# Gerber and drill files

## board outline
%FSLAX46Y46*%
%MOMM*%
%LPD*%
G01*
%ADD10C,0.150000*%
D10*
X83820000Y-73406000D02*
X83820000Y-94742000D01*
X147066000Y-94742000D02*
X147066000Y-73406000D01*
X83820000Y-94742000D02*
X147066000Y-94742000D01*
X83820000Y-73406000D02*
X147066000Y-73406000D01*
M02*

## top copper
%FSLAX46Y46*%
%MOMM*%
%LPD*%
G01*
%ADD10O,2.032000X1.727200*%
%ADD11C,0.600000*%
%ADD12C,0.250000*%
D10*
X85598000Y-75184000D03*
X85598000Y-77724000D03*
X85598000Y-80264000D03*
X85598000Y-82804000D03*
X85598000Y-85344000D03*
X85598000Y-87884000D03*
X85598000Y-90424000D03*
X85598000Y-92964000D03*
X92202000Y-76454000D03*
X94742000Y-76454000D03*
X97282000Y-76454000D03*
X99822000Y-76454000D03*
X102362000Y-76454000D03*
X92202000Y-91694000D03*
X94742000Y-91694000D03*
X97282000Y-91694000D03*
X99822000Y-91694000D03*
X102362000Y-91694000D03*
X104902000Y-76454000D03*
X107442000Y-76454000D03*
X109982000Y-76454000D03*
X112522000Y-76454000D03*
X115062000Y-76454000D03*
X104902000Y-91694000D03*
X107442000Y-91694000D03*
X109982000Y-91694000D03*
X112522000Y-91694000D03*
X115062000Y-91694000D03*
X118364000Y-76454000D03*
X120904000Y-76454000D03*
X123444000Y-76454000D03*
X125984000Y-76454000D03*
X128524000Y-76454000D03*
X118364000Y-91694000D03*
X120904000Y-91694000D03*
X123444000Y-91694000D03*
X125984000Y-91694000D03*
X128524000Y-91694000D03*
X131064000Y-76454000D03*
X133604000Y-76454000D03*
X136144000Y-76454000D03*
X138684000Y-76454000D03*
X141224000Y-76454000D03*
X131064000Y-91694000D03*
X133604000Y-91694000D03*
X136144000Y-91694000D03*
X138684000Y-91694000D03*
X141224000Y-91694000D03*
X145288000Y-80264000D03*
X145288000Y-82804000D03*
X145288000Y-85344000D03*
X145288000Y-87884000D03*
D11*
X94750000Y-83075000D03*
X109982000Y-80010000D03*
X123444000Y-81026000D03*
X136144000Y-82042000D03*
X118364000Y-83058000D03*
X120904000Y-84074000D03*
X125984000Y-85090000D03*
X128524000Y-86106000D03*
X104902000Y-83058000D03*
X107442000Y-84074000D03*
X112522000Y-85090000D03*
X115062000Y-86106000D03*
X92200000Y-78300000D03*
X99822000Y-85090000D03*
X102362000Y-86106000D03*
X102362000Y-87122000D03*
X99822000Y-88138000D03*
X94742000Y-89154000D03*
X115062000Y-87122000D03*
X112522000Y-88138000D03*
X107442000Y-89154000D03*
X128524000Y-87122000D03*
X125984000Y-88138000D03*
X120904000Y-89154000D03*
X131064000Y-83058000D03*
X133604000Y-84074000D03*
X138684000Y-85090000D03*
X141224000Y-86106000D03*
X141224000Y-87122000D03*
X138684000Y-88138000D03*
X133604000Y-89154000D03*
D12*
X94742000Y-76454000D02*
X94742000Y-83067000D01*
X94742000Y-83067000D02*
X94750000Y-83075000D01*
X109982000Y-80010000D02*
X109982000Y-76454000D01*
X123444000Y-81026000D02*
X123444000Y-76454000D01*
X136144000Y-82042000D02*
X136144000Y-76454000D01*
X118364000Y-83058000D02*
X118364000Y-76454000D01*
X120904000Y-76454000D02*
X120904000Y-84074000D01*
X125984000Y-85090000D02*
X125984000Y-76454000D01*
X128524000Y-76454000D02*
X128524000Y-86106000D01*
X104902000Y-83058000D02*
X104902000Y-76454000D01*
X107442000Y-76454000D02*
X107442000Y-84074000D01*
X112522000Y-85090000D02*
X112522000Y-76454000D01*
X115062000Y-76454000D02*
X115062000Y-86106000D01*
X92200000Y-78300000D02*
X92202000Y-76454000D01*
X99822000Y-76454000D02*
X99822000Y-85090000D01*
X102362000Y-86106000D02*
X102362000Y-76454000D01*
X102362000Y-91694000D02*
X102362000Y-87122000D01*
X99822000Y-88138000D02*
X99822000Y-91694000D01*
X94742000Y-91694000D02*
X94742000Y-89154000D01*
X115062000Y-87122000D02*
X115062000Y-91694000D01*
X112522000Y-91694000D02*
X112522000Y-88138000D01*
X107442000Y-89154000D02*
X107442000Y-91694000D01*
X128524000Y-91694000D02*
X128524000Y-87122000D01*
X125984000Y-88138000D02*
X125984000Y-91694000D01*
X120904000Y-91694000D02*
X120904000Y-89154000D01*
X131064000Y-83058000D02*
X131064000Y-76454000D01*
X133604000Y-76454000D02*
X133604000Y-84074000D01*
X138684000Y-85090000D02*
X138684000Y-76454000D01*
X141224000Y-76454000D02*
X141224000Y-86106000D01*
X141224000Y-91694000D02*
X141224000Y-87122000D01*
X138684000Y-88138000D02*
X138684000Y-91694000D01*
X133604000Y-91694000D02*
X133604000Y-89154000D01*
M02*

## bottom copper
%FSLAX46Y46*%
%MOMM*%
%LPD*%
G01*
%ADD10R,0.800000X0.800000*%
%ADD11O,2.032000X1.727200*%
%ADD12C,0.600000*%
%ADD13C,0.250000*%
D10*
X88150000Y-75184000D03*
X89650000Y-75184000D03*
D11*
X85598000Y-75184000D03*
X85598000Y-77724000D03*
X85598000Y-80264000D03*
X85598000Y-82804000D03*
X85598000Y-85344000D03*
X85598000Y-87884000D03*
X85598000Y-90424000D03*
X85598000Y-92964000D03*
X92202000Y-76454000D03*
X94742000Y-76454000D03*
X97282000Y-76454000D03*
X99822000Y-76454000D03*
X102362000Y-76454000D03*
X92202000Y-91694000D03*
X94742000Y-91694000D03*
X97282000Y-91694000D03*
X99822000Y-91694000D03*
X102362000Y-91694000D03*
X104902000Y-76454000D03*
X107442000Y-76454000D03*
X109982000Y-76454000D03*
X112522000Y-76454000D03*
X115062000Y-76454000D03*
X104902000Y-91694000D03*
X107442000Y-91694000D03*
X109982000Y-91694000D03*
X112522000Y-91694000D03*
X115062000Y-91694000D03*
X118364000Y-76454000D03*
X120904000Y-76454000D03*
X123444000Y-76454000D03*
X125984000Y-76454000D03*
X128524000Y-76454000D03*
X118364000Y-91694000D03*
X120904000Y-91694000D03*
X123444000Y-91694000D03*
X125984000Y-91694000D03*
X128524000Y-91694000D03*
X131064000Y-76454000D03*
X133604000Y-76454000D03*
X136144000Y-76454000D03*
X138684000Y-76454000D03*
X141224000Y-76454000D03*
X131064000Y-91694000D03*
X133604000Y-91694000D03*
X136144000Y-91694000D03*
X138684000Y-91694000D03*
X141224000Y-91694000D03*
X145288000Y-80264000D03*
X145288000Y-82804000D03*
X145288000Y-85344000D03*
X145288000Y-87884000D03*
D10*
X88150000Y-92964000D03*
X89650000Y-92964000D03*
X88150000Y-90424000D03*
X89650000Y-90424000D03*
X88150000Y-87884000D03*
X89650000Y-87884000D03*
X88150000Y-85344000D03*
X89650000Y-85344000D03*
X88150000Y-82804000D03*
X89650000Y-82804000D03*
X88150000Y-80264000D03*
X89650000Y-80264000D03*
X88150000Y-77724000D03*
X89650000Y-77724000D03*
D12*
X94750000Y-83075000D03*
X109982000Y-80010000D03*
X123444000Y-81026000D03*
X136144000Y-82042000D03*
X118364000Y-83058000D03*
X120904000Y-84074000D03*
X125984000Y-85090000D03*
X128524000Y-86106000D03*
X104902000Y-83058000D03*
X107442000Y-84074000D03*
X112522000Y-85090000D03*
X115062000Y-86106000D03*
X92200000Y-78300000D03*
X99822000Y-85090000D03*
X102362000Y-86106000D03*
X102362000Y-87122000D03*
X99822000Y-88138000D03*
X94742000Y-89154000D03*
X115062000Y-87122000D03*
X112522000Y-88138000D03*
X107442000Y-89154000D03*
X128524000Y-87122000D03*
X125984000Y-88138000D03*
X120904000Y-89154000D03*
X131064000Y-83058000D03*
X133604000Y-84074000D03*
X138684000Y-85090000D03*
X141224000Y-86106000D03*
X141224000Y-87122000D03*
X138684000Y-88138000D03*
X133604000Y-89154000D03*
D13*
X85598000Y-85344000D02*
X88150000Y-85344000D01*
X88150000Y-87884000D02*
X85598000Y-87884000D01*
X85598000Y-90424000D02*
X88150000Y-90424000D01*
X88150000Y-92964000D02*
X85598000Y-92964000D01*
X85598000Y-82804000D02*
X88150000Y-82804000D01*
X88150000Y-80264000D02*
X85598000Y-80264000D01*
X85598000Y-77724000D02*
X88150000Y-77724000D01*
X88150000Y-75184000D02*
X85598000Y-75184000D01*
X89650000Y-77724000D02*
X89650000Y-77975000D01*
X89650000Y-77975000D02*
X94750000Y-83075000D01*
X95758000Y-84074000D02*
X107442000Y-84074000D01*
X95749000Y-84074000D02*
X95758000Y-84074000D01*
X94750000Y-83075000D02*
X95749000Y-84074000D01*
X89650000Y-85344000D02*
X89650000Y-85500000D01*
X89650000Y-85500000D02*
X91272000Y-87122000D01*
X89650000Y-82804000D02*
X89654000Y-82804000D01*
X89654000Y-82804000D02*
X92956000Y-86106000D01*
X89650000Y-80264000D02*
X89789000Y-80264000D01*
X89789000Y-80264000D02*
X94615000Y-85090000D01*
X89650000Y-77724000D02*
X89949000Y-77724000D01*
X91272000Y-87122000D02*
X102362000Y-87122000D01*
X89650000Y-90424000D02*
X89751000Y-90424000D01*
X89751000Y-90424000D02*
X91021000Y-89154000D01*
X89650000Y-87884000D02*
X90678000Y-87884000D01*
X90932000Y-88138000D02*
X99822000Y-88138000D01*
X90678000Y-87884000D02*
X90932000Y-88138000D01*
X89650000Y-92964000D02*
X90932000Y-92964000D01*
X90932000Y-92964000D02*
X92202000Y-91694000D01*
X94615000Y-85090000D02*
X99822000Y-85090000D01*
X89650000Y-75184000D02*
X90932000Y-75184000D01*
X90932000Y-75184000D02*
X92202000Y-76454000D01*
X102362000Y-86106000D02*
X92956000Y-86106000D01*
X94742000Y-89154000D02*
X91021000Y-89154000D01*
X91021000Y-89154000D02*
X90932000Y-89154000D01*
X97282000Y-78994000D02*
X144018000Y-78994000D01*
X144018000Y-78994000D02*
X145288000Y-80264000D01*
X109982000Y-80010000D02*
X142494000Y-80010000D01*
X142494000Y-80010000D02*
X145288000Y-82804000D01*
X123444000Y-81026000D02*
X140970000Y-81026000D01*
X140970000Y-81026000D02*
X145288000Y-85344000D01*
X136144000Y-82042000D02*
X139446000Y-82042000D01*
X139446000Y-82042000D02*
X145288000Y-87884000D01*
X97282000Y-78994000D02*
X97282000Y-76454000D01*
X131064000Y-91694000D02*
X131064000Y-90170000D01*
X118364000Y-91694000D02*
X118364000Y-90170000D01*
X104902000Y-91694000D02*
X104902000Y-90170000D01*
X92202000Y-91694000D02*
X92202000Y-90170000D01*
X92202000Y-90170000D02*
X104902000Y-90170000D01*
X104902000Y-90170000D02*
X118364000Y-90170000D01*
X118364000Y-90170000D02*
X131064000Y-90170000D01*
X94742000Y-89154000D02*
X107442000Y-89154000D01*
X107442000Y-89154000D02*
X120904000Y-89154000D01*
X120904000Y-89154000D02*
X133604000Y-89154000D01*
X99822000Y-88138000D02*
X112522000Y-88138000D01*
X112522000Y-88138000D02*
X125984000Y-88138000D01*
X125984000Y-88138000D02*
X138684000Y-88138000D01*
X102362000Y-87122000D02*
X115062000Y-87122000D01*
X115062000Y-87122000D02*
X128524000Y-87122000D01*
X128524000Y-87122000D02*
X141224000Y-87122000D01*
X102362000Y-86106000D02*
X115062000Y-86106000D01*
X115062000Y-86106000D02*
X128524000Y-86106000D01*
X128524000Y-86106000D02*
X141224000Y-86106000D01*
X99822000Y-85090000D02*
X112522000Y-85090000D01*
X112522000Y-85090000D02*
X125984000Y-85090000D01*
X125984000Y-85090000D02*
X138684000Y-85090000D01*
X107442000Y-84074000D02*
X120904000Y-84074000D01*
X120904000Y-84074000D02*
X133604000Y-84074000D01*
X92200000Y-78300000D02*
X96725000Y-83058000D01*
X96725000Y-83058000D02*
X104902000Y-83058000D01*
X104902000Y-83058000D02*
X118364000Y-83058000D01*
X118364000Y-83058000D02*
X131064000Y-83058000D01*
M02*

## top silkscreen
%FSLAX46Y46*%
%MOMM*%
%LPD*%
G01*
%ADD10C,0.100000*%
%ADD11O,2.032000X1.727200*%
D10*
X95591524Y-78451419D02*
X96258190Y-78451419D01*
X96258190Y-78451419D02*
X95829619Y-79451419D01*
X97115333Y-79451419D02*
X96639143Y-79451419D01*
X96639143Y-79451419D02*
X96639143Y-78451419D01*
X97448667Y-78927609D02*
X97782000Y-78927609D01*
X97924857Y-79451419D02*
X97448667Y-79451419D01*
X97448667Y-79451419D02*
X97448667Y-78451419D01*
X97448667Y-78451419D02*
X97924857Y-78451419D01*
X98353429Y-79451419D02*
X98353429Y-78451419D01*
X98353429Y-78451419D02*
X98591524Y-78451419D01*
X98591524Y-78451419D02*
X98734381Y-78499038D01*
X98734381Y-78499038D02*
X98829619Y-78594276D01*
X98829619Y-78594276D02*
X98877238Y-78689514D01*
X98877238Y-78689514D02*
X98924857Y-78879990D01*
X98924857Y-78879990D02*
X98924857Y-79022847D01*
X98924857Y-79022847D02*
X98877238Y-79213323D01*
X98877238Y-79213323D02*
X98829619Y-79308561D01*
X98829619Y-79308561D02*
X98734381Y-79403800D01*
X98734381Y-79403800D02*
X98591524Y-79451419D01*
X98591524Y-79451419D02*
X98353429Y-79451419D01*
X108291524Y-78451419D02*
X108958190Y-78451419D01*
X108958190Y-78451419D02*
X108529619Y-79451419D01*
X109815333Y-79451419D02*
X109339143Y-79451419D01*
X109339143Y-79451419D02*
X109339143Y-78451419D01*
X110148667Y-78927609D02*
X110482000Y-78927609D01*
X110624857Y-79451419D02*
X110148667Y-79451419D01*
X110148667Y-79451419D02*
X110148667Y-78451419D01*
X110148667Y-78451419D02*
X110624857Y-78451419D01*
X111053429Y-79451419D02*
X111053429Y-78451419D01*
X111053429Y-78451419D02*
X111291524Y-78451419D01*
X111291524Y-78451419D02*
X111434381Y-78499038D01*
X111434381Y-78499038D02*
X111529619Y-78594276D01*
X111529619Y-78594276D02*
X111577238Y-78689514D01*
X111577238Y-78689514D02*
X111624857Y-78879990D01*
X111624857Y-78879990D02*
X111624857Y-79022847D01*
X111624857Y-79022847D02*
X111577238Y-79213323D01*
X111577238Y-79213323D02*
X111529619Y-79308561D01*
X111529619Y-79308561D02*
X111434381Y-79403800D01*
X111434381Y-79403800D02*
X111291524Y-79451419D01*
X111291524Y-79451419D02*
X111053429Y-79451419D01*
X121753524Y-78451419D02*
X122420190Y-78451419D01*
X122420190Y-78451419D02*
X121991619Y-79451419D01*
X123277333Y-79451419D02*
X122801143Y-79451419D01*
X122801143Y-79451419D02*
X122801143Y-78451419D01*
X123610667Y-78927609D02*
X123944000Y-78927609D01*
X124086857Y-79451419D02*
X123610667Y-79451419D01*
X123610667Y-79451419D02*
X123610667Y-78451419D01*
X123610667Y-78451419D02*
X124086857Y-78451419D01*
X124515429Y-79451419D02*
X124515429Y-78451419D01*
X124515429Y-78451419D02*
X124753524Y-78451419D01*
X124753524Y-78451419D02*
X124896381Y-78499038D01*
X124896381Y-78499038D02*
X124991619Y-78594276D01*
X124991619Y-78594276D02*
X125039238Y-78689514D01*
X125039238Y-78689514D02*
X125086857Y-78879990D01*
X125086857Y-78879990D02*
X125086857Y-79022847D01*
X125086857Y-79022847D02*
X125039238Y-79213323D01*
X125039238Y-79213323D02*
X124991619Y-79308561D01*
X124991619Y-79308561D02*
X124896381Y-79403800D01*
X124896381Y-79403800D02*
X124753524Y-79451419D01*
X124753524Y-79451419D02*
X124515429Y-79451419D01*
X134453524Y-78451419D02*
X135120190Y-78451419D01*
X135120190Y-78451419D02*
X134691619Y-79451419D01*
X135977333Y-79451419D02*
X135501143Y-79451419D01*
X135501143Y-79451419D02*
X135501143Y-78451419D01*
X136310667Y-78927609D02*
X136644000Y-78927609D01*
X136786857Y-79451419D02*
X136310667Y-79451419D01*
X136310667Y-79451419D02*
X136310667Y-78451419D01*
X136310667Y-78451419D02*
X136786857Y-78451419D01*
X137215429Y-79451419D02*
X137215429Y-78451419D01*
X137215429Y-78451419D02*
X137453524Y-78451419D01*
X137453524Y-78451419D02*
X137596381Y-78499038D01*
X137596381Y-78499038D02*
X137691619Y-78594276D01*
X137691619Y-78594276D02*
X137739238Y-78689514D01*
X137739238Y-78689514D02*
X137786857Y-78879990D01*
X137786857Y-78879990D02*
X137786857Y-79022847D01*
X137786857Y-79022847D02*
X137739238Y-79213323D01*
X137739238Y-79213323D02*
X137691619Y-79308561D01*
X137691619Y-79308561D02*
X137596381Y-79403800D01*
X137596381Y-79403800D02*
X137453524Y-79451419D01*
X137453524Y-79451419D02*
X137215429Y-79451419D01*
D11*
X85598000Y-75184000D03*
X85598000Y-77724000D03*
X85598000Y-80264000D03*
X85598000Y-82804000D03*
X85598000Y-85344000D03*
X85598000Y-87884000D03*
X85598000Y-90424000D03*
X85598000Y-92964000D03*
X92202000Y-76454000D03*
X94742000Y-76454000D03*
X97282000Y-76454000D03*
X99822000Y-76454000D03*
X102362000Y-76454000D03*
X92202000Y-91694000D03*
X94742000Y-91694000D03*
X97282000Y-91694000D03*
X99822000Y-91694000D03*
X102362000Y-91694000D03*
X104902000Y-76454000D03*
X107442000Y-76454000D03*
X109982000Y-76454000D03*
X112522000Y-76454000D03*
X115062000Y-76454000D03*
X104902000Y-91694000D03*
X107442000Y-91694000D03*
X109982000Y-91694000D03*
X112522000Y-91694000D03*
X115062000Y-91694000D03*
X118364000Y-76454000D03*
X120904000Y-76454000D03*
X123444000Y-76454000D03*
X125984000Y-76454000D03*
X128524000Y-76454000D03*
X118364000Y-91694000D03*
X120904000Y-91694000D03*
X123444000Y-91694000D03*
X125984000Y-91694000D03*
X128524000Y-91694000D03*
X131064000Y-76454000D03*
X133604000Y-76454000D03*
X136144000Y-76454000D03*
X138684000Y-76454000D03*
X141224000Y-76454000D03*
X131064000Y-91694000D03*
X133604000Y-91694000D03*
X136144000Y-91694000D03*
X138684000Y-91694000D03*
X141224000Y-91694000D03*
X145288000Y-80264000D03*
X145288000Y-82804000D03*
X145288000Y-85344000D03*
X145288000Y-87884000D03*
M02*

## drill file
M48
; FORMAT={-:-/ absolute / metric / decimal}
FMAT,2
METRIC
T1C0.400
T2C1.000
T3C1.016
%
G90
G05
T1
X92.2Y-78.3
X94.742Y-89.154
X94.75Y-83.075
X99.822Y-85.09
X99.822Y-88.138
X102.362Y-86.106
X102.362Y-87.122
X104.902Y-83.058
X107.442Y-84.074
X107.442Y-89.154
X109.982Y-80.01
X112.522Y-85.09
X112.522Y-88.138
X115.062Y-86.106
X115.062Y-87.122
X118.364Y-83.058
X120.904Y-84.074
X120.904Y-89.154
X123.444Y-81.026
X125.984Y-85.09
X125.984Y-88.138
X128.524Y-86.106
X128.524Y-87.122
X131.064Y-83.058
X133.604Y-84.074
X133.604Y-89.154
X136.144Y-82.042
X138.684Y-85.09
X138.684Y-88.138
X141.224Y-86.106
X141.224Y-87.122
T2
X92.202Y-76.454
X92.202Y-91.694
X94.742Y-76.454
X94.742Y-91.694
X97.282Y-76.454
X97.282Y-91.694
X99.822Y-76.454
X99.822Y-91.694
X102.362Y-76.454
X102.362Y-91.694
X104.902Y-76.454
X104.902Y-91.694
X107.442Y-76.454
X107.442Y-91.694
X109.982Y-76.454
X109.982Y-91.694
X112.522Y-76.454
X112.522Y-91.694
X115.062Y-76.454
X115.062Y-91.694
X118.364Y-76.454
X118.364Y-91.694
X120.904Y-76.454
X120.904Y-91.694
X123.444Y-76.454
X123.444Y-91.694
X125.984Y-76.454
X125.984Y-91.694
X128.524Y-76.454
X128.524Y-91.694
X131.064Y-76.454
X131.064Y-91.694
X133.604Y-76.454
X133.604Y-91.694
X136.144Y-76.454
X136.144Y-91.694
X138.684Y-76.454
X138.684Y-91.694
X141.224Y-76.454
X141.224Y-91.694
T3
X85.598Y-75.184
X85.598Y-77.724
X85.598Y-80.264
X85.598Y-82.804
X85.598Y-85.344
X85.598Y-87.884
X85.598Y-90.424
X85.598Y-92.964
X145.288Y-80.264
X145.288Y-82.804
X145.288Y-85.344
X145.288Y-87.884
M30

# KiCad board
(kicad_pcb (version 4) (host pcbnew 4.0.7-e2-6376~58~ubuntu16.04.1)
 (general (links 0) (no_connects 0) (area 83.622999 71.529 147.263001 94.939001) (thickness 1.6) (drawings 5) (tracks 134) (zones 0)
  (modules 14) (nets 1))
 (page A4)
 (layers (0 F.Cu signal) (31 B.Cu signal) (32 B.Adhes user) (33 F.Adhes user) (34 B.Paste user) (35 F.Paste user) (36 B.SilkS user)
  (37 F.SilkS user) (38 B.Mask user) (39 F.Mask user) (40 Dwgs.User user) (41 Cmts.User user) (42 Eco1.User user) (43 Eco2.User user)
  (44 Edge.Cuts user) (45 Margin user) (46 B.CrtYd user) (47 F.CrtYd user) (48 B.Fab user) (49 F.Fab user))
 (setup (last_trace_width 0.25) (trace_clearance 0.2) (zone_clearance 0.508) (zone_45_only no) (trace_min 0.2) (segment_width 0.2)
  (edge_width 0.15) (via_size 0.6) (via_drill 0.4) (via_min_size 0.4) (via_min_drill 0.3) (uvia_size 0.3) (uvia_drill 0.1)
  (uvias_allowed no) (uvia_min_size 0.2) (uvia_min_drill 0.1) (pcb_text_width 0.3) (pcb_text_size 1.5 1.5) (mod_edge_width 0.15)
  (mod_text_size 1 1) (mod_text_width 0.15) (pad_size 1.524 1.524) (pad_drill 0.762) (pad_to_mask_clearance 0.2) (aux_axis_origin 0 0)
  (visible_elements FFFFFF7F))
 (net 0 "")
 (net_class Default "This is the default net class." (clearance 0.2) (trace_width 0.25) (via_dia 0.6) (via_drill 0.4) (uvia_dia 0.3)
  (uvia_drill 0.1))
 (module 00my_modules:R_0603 (layer B.Cu) (at 88.9 75.184)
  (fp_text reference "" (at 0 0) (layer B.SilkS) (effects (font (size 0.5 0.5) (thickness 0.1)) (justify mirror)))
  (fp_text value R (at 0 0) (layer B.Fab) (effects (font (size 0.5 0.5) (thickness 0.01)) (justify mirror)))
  (pad 1 smd rect (at -0.75 0) (size 0.8 0.8) (layers B.Cu B.Paste B.Mask))
  (pad 2 smd rect (at 0.75 0) (size 0.8 0.8) (layers B.Cu B.Paste B.Mask)))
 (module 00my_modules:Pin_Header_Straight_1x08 (layer F.Cu) (at 85.598 75.184)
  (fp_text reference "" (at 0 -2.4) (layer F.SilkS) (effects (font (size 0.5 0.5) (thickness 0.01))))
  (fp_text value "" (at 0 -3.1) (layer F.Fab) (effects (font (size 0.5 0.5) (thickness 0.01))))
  (pad 1 thru_hole oval (at 0 0) (size 2.032 1.7272) (drill 1.016) (layers *.Cu *.Mask F.SilkS))
  (pad 2 thru_hole oval (at 0 2.54) (size 2.032 1.7272) (drill 1.016) (layers *.Cu *.Mask F.SilkS))
  (pad 3 thru_hole oval (at 0 5.08) (size 2.032 1.7272) (drill 1.016) (layers *.Cu *.Mask F.SilkS))
  (pad 4 thru_hole oval (at 0 7.62) (size 2.032 1.7272) (drill 1.016) (layers *.Cu *.Mask F.SilkS))
  (pad 5 thru_hole oval (at 0 10.16) (size 2.032 1.7272) (drill 1.016) (layers *.Cu *.Mask F.SilkS))
  (pad 6 thru_hole oval (at 0 12.7) (size 2.032 1.7272) (drill 1.016) (layers *.Cu *.Mask F.SilkS))
  (pad 7 thru_hole oval (at 0 15.24) (size 2.032 1.7272) (drill 1.016) (layers *.Cu *.Mask F.SilkS))
  (pad 8 thru_hole oval (at 0 17.78) (size 2.032 1.7272) (drill 1.016) (layers *.Cu *.Mask F.SilkS)))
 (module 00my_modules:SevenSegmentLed (layer F.Cu) (at 92.202 76.454)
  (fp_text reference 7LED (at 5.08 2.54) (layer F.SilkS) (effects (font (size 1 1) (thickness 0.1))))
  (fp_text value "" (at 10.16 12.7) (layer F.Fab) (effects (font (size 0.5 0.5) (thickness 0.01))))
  (pad 10 thru_hole oval (at 0 0) (size 2.032 1.7272) (drill 1) (layers *.Cu *.Mask F.SilkS))
  (pad 9 thru_hole oval (at 2.54 0) (size 2.032 1.7272) (drill 1) (layers *.Cu *.Mask F.SilkS))
  (pad 8 thru_hole oval (at 5.08 0) (size 2.032 1.7272) (drill 1) (layers *.Cu *.Mask F.SilkS))
  (pad 7 thru_hole oval (at 7.62 0) (size 2.032 1.7272) (drill 1) (layers *.Cu *.Mask F.SilkS))
  (pad 6 thru_hole oval (at 10.16 0) (size 2.032 1.7272) (drill 1) (layers *.Cu *.Mask F.SilkS))
  (pad 1 thru_hole oval (at 0 15.24) (size 2.032 1.7272) (drill 1) (layers *.Cu *.Mask F.SilkS))
  (pad 2 thru_hole oval (at 2.54 15.24) (size 2.032 1.7272) (drill 1) (layers *.Cu *.Mask F.SilkS))
  (pad 3 thru_hole oval (at 5.08 15.24) (size 2.032 1.7272) (drill 1) (layers *.Cu *.Mask F.SilkS))
  (pad 4 thru_hole oval (at 7.62 15.24) (size 2.032 1.7272) (drill 1) (layers *.Cu *.Mask F.SilkS))
  (pad 5 thru_hole oval (at 10.16 15.24) (size 2.032 1.7272) (drill 1) (layers *.Cu *.Mask F.SilkS)))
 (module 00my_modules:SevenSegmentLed (layer F.Cu) (at 104.902 76.454)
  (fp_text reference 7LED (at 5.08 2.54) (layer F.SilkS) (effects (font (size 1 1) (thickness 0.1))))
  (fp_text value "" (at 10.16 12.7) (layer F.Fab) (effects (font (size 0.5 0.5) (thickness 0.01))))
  (pad 10 thru_hole oval (at 0 0) (size 2.032 1.7272) (drill 1) (layers *.Cu *.Mask F.SilkS))
  (pad 9 thru_hole oval (at 2.54 0) (size 2.032 1.7272) (drill 1) (layers *.Cu *.Mask F.SilkS))
  (pad 8 thru_hole oval (at 5.08 0) (size 2.032 1.7272) (drill 1) (layers *.Cu *.Mask F.SilkS))
  (pad 7 thru_hole oval (at 7.62 0) (size 2.032 1.7272) (drill 1) (layers *.Cu *.Mask F.SilkS))
  (pad 6 thru_hole oval (at 10.16 0) (size 2.032 1.7272) (drill 1) (layers *.Cu *.Mask F.SilkS))
  (pad 1 thru_hole oval (at 0 15.24) (size 2.032 1.7272) (drill 1) (layers *.Cu *.Mask F.SilkS))
  (pad 2 thru_hole oval (at 2.54 15.24) (size 2.032 1.7272) (drill 1) (layers *.Cu *.Mask F.SilkS))
  (pad 3 thru_hole oval (at 5.08 15.24) (size 2.032 1.7272) (drill 1) (layers *.Cu *.Mask F.SilkS))
  (pad 4 thru_hole oval (at 7.62 15.24) (size 2.032 1.7272) (drill 1) (layers *.Cu *.Mask F.SilkS))
  (pad 5 thru_hole oval (at 10.16 15.24) (size 2.032 1.7272) (drill 1) (layers *.Cu *.Mask F.SilkS)))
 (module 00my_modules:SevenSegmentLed (layer F.Cu) (at 118.364 76.454)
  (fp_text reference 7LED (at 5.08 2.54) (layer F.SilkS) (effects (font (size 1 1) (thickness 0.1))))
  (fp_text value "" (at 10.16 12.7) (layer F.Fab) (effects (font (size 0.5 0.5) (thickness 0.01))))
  (pad 10 thru_hole oval (at 0 0) (size 2.032 1.7272) (drill 1) (layers *.Cu *.Mask F.SilkS))
  (pad 9 thru_hole oval (at 2.54 0) (size 2.032 1.7272) (drill 1) (layers *.Cu *.Mask F.SilkS))
  (pad 8 thru_hole oval (at 5.08 0) (size 2.032 1.7272) (drill 1) (layers *.Cu *.Mask F.SilkS))
  (pad 7 thru_hole oval (at 7.62 0) (size 2.032 1.7272) (drill 1) (layers *.Cu *.Mask F.SilkS))
  (pad 6 thru_hole oval (at 10.16 0) (size 2.032 1.7272) (drill 1) (layers *.Cu *.Mask F.SilkS))
  (pad 1 thru_hole oval (at 0 15.24) (size 2.032 1.7272) (drill 1) (layers *.Cu *.Mask F.SilkS))
  (pad 2 thru_hole oval (at 2.54 15.24) (size 2.032 1.7272) (drill 1) (layers *.Cu *.Mask F.SilkS))
  (pad 3 thru_hole oval (at 5.08 15.24) (size 2.032 1.7272) (drill 1) (layers *.Cu *.Mask F.SilkS))
  (pad 4 thru_hole oval (at 7.62 15.24) (size 2.032 1.7272) (drill 1) (layers *.Cu *.Mask F.SilkS))
  (pad 5 thru_hole oval (at 10.16 15.24) (size 2.032 1.7272) (drill 1) (layers *.Cu *.Mask F.SilkS)))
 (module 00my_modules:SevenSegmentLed (layer F.Cu) (at 131.064 76.454)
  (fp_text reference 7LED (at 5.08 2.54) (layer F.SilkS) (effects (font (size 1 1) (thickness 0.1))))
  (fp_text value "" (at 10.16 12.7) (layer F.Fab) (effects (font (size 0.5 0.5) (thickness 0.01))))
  (pad 10 thru_hole oval (at 0 0) (size 2.032 1.7272) (drill 1) (layers *.Cu *.Mask F.SilkS))
  (pad 9 thru_hole oval (at 2.54 0) (size 2.032 1.7272) (drill 1) (layers *.Cu *.Mask F.SilkS))
  (pad 8 thru_hole oval (at 5.08 0) (size 2.032 1.7272) (drill 1) (layers *.Cu *.Mask F.SilkS))
  (pad 7 thru_hole oval (at 7.62 0) (size 2.032 1.7272) (drill 1) (layers *.Cu *.Mask F.SilkS))
  (pad 6 thru_hole oval (at 10.16 0) (size 2.032 1.7272) (drill 1) (layers *.Cu *.Mask F.SilkS))
  (pad 1 thru_hole oval (at 0 15.24) (size 2.032 1.7272) (drill 1) (layers *.Cu *.Mask F.SilkS))
  (pad 2 thru_hole oval (at 2.54 15.24) (size 2.032 1.7272) (drill 1) (layers *.Cu *.Mask F.SilkS))
  (pad 3 thru_hole oval (at 5.08 15.24) (size 2.032 1.7272) (drill 1) (layers *.Cu *.Mask F.SilkS))
  (pad 4 thru_hole oval (at 7.62 15.24) (size 2.032 1.7272) (drill 1) (layers *.Cu *.Mask F.SilkS))
  (pad 5 thru_hole oval (at 10.16 15.24) (size 2.032 1.7272) (drill 1) (layers *.Cu *.Mask F.SilkS)))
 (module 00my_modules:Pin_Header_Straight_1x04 (layer F.Cu) (at 145.288 80.264)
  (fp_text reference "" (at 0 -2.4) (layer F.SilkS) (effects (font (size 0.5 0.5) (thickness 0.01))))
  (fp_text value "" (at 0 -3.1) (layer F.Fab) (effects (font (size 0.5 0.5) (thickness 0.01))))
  (pad 1 thru_hole oval (at 0 0) (size 2.032 1.7272) (drill 1.016) (layers *.Cu *.Mask F.SilkS))
  (pad 2 thru_hole oval (at 0 2.54) (size 2.032 1.7272) (drill 1.016) (layers *.Cu *.Mask F.SilkS))
  (pad 3 thru_hole oval (at 0 5.08) (size 2.032 1.7272) (drill 1.016) (layers *.Cu *.Mask F.SilkS))
  (pad 4 thru_hole oval (at 0 7.62) (size 2.032 1.7272) (drill 1.016) (layers *.Cu *.Mask F.SilkS)))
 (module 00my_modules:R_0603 (layer B.Cu) (at 88.9 92.964)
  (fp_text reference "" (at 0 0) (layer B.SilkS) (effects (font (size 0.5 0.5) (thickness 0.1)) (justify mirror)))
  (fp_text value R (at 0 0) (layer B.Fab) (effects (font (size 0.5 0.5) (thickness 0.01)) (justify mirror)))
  (pad 1 smd rect (at -0.75 0) (size 0.8 0.8) (layers B.Cu B.Paste B.Mask))
  (pad 2 smd rect (at 0.75 0) (size 0.8 0.8) (layers B.Cu B.Paste B.Mask)))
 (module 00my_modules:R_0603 (layer B.Cu) (at 88.9 90.424)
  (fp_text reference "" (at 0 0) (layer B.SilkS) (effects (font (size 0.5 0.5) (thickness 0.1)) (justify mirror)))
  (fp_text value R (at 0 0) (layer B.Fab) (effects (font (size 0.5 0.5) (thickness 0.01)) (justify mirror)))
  (pad 1 smd rect (at -0.75 0) (size 0.8 0.8) (layers B.Cu B.Paste B.Mask))
  (pad 2 smd rect (at 0.75 0) (size 0.8 0.8) (layers B.Cu B.Paste B.Mask)))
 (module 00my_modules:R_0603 (layer B.Cu) (at 88.9 87.884)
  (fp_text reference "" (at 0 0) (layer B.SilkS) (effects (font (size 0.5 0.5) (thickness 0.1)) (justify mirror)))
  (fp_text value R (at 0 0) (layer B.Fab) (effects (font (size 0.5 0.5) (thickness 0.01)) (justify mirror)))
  (pad 1 smd rect (at -0.75 0) (size 0.8 0.8) (layers B.Cu B.Paste B.Mask))
  (pad 2 smd rect (at 0.75 0) (size 0.8 0.8) (layers B.Cu B.Paste B.Mask)))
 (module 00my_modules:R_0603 (layer B.Cu) (at 88.9 85.344)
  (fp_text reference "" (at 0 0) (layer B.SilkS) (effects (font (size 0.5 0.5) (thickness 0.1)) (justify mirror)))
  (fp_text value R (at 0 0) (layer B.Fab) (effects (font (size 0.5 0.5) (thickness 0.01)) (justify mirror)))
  (pad 1 smd rect (at -0.75 0) (size 0.8 0.8) (layers B.Cu B.Paste B.Mask))
  (pad 2 smd rect (at 0.75 0) (size 0.8 0.8) (layers B.Cu B.Paste B.Mask)))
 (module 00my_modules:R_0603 (layer B.Cu) (at 88.9 82.804)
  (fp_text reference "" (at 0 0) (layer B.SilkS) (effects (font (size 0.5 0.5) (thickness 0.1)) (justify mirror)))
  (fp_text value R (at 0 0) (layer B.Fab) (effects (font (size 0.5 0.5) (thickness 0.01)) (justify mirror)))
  (pad 1 smd rect (at -0.75 0) (size 0.8 0.8) (layers B.Cu B.Paste B.Mask))
  (pad 2 smd rect (at 0.75 0) (size 0.8 0.8) (layers B.Cu B.Paste B.Mask)))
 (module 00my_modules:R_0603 (layer B.Cu) (at 88.9 80.264)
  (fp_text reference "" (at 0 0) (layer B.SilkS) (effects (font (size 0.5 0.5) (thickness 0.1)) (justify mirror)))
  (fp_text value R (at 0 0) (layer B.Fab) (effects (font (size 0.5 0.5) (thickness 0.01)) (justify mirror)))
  (pad 1 smd rect (at -0.75 0) (size 0.8 0.8) (layers B.Cu B.Paste B.Mask))
  (pad 2 smd rect (at 0.75 0) (size 0.8 0.8) (layers B.Cu B.Paste B.Mask)))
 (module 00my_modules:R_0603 (layer B.Cu) (at 88.9 77.724)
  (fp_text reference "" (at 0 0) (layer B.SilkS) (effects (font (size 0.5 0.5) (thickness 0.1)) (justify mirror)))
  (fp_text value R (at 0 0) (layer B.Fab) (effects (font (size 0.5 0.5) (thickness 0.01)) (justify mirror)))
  (pad 1 smd rect (at -0.75 0) (size 0.8 0.8) (layers B.Cu B.Paste B.Mask))
  (pad 2 smd rect (at 0.75 0) (size 0.8 0.8) (layers B.Cu B.Paste B.Mask)))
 (gr_line (start 83.82 73.406) (end 83.82 94.742) (angle 90) (layer Edge.Cuts) (width 0.15))
 (gr_line (start 147.066 94.742) (end 147.066 73.406) (angle 90) (layer Edge.Cuts) (width 0.15))
 (gr_line (start 83.82 94.742) (end 147.066 94.742) (angle 90) (layer Edge.Cuts) (width 0.15))
 (gr_line (start 83.82 73.406) (end 147.066 73.406) (angle 90) (layer Edge.Cuts) (width 0.15))
 (segment (start 85.598 85.344) (end 88.15 85.344) (width 0.25) (layer B.Cu) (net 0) (status C00000))
 (segment (start 88.15 87.884) (end 85.598 87.884) (width 0.25) (layer B.Cu) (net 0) (status C00000))
 (segment (start 85.598 90.424) (end 88.15 90.424) (width 0.25) (layer B.Cu) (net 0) (status C00000))
 (segment (start 88.15 92.964) (end 85.598 92.964) (width 0.25) (layer B.Cu) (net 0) (status C00000))
 (segment (start 85.598 82.804) (end 88.15 82.804) (width 0.25) (layer B.Cu) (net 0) (status C00000))
 (segment (start 88.15 80.264) (end 85.598 80.264) (width 0.25) (layer B.Cu) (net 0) (status C00000))
 (segment (start 85.598 77.724) (end 88.15 77.724) (width 0.25) (layer B.Cu) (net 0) (status C00000))
 (segment (start 88.15 75.184) (end 85.598 75.184) (width 0.25) (layer B.Cu) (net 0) (status C00000))
 (segment (start 89.65 77.724) (end 89.65 77.975) (width 0.25) (layer B.Cu) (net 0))
 (segment (start 89.65 77.975) (end 94.75 83.075) (width 0.25) (layer B.Cu) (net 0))
 (segment (start 94.742 76.454) (end 94.742 83.067) (width 0.25) (layer F.Cu) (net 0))
 (segment (start 95.758 84.074) (end 107.442 84.074) (width 0.25) (layer B.Cu) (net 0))
 (segment (start 95.749 84.074) (end 95.758 84.074) (width 0.25) (layer B.Cu) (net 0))
 (segment (start 94.75 83.075) (end 95.749 84.074) (width 0.25) (layer B.Cu) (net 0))
 (via (at 94.75 83.075) (size 0.6) (drill 0.4) (layers F.Cu B.Cu) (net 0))
 (segment (start 94.742 83.067) (end 94.75 83.075) (width 0.25) (layer F.Cu) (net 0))
 (segment (start 89.65 85.344) (end 89.65 85.5) (width 0.25) (layer B.Cu) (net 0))
 (segment (start 89.65 85.5) (end 91.272 87.122) (width 0.25) (layer B.Cu) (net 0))
 (segment (start 89.65 82.804) (end 89.654 82.804) (width 0.25) (layer B.Cu) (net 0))
 (segment (start 89.654 82.804) (end 92.956 86.106) (width 0.25) (layer B.Cu) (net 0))
 (segment (start 89.65 80.264) (end 89.789 80.264) (width 0.25) (layer B.Cu) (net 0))
 (segment (start 89.789 80.264) (end 94.615 85.09) (width 0.25) (layer B.Cu) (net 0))
 (segment (start 89.65 77.724) (end 89.949 77.724) (width 0.25) (layer B.Cu) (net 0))
 (segment (start 91.272 87.122) (end 102.362 87.122) (width 0.25) (layer B.Cu) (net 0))
 (segment (start 89.65 90.424) (end 89.751 90.424) (width 0.25) (layer B.Cu) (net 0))
 (segment (start 89.751 90.424) (end 91.021 89.154) (width 0.25) (layer B.Cu) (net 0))
 (segment (start 89.65 87.884) (end 90.678 87.884) (width 0.25) (layer B.Cu) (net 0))
 (segment (start 90.932 88.138) (end 99.822 88.138) (width 0.25) (layer B.Cu) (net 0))
 (segment (start 90.678 87.884) (end 90.932 88.138) (width 0.25) (layer B.Cu) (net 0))
 (segment (start 89.65 92.964) (end 90.932 92.964) (width 0.25) (layer B.Cu) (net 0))
 (segment (start 90.932 92.964) (end 92.202 91.694) (width 0.25) (layer B.Cu) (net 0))
 (segment (start 94.615 85.09) (end 99.822 85.09) (width 0.25) (layer B.Cu) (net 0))
 (segment (start 89.65 75.184) (end 90.932 75.184) (width 0.25) (layer B.Cu) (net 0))
 (segment (start 90.932 75.184) (end 92.202 76.454) (width 0.25) (layer B.Cu) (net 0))
 (segment (start 102.362 86.106) (end 92.956 86.106) (width 0.25) (layer B.Cu) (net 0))
 (segment (start 94.742 89.154) (end 91.021 89.154) (width 0.25) (layer B.Cu) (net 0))
 (segment (start 91.021 89.154) (end 90.932 89.154) (width 0.25) (layer B.Cu) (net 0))
 (segment (start 97.282 78.994) (end 144.018 78.994) (width 0.25) (layer B.Cu) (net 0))
 (segment (start 144.018 78.994) (end 145.288 80.264) (width 0.25) (layer B.Cu) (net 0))
 (segment (start 109.982 80.01) (end 142.494 80.01) (width 0.25) (layer B.Cu) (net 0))
 (segment (start 142.494 80.01) (end 145.288 82.804) (width 0.25) (layer B.Cu) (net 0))
 (segment (start 123.444 81.026) (end 140.97 81.026) (width 0.25) (layer B.Cu) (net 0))
 (segment (start 140.97 81.026) (end 145.288 85.344) (width 0.25) (layer B.Cu) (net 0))
 (segment (start 136.144 82.042) (end 139.446 82.042) (width 0.25) (layer B.Cu) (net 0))
 (segment (start 139.446 82.042) (end 145.288 87.884) (width 0.25) (layer B.Cu) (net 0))
 (segment (start 97.282 78.994) (end 97.282 76.454) (width 0.25) (layer B.Cu) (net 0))
 (via (at 109.982 80.01) (size 0.6) (drill 0.4) (layers F.Cu B.Cu) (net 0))
 (segment (start 109.982 80.01) (end 109.982 76.454) (width 0.25) (layer F.Cu) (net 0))
 (segment (start 123.444 81.026) (end 123.444 76.454) (width 0.25) (layer F.Cu) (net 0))
 (via (at 123.444 81.026) (size 0.6) (drill 0.4) (layers F.Cu B.Cu) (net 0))
 (via (at 136.144 82.042) (size 0.6) (drill 0.4) (layers F.Cu B.Cu) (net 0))
 (segment (start 136.144 82.042) (end 136.144 76.454) (width 0.25) (layer F.Cu) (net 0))
 (via (at 118.364 83.058) (size 0.6) (drill 0.4) (layers F.Cu B.Cu) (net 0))
 (segment (start 118.364 83.058) (end 118.364 76.454) (width 0.25) (layer F.Cu) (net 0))
 (segment (start 120.904 76.454) (end 120.904 84.074) (width 0.25) (layer F.Cu) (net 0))
 (via (at 120.904 84.074) (size 0.6) (drill 0.4) (layers F.Cu B.Cu) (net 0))
 (via (at 125.984 85.09) (size 0.6) (drill 0.4) (layers F.Cu B.Cu) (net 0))
 (segment (start 125.984 85.09) (end 125.984 76.454) (width 0.25) (layer F.Cu) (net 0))
 (segment (start 128.524 76.454) (end 128.524 86.106) (width 0.25) (layer F.Cu) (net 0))
 (via (at 128.524 86.106) (size 0.6) (drill 0.4) (layers F.Cu B.Cu) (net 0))
 (via (at 104.902 83.058) (size 0.6) (drill 0.4) (layers F.Cu B.Cu) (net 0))
 (segment (start 104.902 83.058) (end 104.902 76.454) (width 0.25) (layer F.Cu) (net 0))
 (segment (start 107.442 76.454) (end 107.442 84.074) (width 0.25) (layer F.Cu) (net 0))
 (via (at 107.442 84.074) (size 0.6) (drill 0.4) (layers F.Cu B.Cu) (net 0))
 (via (at 112.522 85.09) (size 0.6) (drill 0.4) (layers F.Cu B.Cu) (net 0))
 (segment (start 112.522 85.09) (end 112.522 76.454) (width 0.25) (layer F.Cu) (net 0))
 (segment (start 115.062 76.454) (end 115.062 86.106) (width 0.25) (layer F.Cu) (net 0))
 (via (at 115.062 86.106) (size 0.6) (drill 0.4) (layers F.Cu B.Cu) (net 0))
 (via (at 92.2 78.3) (size 0.6) (drill 0.4) (layers F.Cu B.Cu) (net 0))
 (segment (start 92.2 78.3) (end 92.202 76.454) (width 0.25) (layer F.Cu) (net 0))
 (segment (start 99.822 76.454) (end 99.822 85.09) (width 0.25) (layer F.Cu) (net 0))
 (via (at 99.822 85.09) (size 0.6) (drill 0.4) (layers F.Cu B.Cu) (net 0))
 (via (at 102.362 86.106) (size 0.6) (drill 0.4) (layers F.Cu B.Cu) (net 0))
 (segment (start 102.362 86.106) (end 102.362 76.454) (width 0.25) (layer F.Cu) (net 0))
 (segment (start 102.362 91.694) (end 102.362 87.122) (width 0.25) (layer F.Cu) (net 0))
 (via (at 102.362 87.122) (size 0.6) (drill 0.4) (layers F.Cu B.Cu) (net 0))
 (via (at 99.822 88.138) (size 0.6) (drill 0.4) (layers F.Cu B.Cu) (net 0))
 (segment (start 99.822 88.138) (end 99.822 91.694) (width 0.25) (layer F.Cu) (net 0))
 (segment (start 94.742 91.694) (end 94.742 89.154) (width 0.25) (layer F.Cu) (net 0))
 (via (at 94.742 89.154) (size 0.6) (drill 0.4) (layers F.Cu B.Cu) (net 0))
 (via (at 115.062 87.122) (size 0.6) (drill 0.4) (layers F.Cu B.Cu) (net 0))
 (segment (start 115.062 87.122) (end 115.062 91.694) (width 0.25) (layer F.Cu) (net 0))
 (segment (start 112.522 91.694) (end 112.522 88.138) (width 0.25) (layer F.Cu) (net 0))
 (via (at 112.522 88.138) (size 0.6) (drill 0.4) (layers F.Cu B.Cu) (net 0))
 (via (at 107.442 89.154) (size 0.6) (drill 0.4) (layers F.Cu B.Cu) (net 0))
 (segment (start 107.442 89.154) (end 107.442 91.694) (width 0.25) (layer F.Cu) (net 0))
 (segment (start 128.524 91.694) (end 128.524 87.122) (width 0.25) (layer F.Cu) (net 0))
 (via (at 128.524 87.122) (size 0.6) (drill 0.4) (layers F.Cu B.Cu) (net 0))
 (via (at 125.984 88.138) (size 0.6) (drill 0.4) (layers F.Cu B.Cu) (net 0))
 (segment (start 125.984 88.138) (end 125.984 91.694) (width 0.25) (layer F.Cu) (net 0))
 (segment (start 120.904 91.694) (end 120.904 89.154) (width 0.25) (layer F.Cu) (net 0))
 (via (at 120.904 89.154) (size 0.6) (drill 0.4) (layers F.Cu B.Cu) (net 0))
 (via (at 131.064 83.058) (size 0.6) (drill 0.4) (layers F.Cu B.Cu) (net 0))
 (segment (start 131.064 83.058) (end 131.064 76.454) (width 0.25) (layer F.Cu) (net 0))
 (segment (start 133.604 76.454) (end 133.604 84.074) (width 0.25) (layer F.Cu) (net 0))
 (via (at 133.604 84.074) (size 0.6) (drill 0.4) (layers F.Cu B.Cu) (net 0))
 (via (at 138.684 85.09) (size 0.6) (drill 0.4) (layers F.Cu B.Cu) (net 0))
 (segment (start 138.684 85.09) (end 138.684 76.454) (width 0.25) (layer F.Cu) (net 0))
 (segment (start 141.224 76.454) (end 141.224 86.106) (width 0.25) (layer F.Cu) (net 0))
 (via (at 141.224 86.106) (size 0.6) (drill 0.4) (layers F.Cu B.Cu) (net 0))
 (segment (start 141.224 91.694) (end 141.224 87.122) (width 0.25) (layer F.Cu) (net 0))
 (via (at 141.224 87.122) (size 0.6) (drill 0.4) (layers F.Cu B.Cu) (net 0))
 (via (at 138.684 88.138) (size 0.6) (drill 0.4) (layers F.Cu B.Cu) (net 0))
 (segment (start 138.684 88.138) (end 138.684 91.694) (width 0.25) (layer F.Cu) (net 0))
 (segment (start 133.604 91.694) (end 133.604 89.154) (width 0.25) (layer F.Cu) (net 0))
 (via (at 133.604 89.154) (size 0.6) (drill 0.4) (layers F.Cu B.Cu) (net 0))
 (segment (start 131.064 91.694) (end 131.064 90.17) (width 0.25) (layer B.Cu) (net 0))
 (segment (start 118.364 91.694) (end 118.364 90.17) (width 0.25) (layer B.Cu) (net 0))
 (segment (start 104.902 91.694) (end 104.902 90.17) (width 0.25) (layer B.Cu) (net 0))
 (segment (start 92.202 91.694) (end 92.202 90.17) (width 0.25) (layer B.Cu) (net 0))
 (segment (start 92.202 90.17) (end 104.902 90.17) (width 0.25) (layer B.Cu) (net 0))
 (segment (start 104.902 90.17) (end 118.364 90.17) (width 0.25) (layer B.Cu) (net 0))
 (segment (start 118.364 90.17) (end 131.064 90.17) (width 0.25) (layer B.Cu) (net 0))
 (segment (start 94.742 89.154) (end 107.442 89.154) (width 0.25) (layer B.Cu) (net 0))
 (segment (start 107.442 89.154) (end 120.904 89.154) (width 0.25) (layer B.Cu) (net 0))
 (segment (start 120.904 89.154) (end 133.604 89.154) (width 0.25) (layer B.Cu) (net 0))
 (segment (start 99.822 88.138) (end 112.522 88.138) (width 0.25) (layer B.Cu) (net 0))
 (segment (start 112.522 88.138) (end 125.984 88.138) (width 0.25) (layer B.Cu) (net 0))
 (segment (start 125.984 88.138) (end 138.684 88.138) (width 0.25) (layer B.Cu) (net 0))
 (segment (start 102.362 87.122) (end 115.062 87.122) (width 0.25) (layer B.Cu) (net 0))
 (segment (start 115.062 87.122) (end 128.524 87.122) (width 0.25) (layer B.Cu) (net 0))
 (segment (start 128.524 87.122) (end 141.224 87.122) (width 0.25) (layer B.Cu) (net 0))
 (segment (start 102.362 86.106) (end 115.062 86.106) (width 0.25) (layer B.Cu) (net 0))
 (segment (start 115.062 86.106) (end 128.524 86.106) (width 0.25) (layer B.Cu) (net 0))
 (segment (start 128.524 86.106) (end 141.224 86.106) (width 0.25) (layer B.Cu) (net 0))
 (segment (start 99.822 85.09) (end 112.522 85.09) (width 0.25) (layer B.Cu) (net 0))
 (segment (start 112.522 85.09) (end 125.984 85.09) (width 0.25) (layer B.Cu) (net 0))
 (segment (start 125.984 85.09) (end 138.684 85.09) (width 0.25) (layer B.Cu) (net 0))
 (segment (start 107.442 84.074) (end 120.904 84.074) (width 0.25) (layer B.Cu) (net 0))
 (segment (start 120.904 84.074) (end 133.604 84.074) (width 0.25) (layer B.Cu) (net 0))
 (segment (start 92.2 78.3) (end 96.725 83.058) (width 0.25) (layer B.Cu) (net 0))
 (segment (start 96.725 83.058) (end 104.902 83.058) (width 0.25) (layer B.Cu) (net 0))
 (segment (start 104.902 83.058) (end 118.364 83.058) (width 0.25) (layer B.Cu) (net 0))
 (segment (start 118.364 83.058) (end 131.064 83.058) (width 0.25) (layer B.Cu) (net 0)))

